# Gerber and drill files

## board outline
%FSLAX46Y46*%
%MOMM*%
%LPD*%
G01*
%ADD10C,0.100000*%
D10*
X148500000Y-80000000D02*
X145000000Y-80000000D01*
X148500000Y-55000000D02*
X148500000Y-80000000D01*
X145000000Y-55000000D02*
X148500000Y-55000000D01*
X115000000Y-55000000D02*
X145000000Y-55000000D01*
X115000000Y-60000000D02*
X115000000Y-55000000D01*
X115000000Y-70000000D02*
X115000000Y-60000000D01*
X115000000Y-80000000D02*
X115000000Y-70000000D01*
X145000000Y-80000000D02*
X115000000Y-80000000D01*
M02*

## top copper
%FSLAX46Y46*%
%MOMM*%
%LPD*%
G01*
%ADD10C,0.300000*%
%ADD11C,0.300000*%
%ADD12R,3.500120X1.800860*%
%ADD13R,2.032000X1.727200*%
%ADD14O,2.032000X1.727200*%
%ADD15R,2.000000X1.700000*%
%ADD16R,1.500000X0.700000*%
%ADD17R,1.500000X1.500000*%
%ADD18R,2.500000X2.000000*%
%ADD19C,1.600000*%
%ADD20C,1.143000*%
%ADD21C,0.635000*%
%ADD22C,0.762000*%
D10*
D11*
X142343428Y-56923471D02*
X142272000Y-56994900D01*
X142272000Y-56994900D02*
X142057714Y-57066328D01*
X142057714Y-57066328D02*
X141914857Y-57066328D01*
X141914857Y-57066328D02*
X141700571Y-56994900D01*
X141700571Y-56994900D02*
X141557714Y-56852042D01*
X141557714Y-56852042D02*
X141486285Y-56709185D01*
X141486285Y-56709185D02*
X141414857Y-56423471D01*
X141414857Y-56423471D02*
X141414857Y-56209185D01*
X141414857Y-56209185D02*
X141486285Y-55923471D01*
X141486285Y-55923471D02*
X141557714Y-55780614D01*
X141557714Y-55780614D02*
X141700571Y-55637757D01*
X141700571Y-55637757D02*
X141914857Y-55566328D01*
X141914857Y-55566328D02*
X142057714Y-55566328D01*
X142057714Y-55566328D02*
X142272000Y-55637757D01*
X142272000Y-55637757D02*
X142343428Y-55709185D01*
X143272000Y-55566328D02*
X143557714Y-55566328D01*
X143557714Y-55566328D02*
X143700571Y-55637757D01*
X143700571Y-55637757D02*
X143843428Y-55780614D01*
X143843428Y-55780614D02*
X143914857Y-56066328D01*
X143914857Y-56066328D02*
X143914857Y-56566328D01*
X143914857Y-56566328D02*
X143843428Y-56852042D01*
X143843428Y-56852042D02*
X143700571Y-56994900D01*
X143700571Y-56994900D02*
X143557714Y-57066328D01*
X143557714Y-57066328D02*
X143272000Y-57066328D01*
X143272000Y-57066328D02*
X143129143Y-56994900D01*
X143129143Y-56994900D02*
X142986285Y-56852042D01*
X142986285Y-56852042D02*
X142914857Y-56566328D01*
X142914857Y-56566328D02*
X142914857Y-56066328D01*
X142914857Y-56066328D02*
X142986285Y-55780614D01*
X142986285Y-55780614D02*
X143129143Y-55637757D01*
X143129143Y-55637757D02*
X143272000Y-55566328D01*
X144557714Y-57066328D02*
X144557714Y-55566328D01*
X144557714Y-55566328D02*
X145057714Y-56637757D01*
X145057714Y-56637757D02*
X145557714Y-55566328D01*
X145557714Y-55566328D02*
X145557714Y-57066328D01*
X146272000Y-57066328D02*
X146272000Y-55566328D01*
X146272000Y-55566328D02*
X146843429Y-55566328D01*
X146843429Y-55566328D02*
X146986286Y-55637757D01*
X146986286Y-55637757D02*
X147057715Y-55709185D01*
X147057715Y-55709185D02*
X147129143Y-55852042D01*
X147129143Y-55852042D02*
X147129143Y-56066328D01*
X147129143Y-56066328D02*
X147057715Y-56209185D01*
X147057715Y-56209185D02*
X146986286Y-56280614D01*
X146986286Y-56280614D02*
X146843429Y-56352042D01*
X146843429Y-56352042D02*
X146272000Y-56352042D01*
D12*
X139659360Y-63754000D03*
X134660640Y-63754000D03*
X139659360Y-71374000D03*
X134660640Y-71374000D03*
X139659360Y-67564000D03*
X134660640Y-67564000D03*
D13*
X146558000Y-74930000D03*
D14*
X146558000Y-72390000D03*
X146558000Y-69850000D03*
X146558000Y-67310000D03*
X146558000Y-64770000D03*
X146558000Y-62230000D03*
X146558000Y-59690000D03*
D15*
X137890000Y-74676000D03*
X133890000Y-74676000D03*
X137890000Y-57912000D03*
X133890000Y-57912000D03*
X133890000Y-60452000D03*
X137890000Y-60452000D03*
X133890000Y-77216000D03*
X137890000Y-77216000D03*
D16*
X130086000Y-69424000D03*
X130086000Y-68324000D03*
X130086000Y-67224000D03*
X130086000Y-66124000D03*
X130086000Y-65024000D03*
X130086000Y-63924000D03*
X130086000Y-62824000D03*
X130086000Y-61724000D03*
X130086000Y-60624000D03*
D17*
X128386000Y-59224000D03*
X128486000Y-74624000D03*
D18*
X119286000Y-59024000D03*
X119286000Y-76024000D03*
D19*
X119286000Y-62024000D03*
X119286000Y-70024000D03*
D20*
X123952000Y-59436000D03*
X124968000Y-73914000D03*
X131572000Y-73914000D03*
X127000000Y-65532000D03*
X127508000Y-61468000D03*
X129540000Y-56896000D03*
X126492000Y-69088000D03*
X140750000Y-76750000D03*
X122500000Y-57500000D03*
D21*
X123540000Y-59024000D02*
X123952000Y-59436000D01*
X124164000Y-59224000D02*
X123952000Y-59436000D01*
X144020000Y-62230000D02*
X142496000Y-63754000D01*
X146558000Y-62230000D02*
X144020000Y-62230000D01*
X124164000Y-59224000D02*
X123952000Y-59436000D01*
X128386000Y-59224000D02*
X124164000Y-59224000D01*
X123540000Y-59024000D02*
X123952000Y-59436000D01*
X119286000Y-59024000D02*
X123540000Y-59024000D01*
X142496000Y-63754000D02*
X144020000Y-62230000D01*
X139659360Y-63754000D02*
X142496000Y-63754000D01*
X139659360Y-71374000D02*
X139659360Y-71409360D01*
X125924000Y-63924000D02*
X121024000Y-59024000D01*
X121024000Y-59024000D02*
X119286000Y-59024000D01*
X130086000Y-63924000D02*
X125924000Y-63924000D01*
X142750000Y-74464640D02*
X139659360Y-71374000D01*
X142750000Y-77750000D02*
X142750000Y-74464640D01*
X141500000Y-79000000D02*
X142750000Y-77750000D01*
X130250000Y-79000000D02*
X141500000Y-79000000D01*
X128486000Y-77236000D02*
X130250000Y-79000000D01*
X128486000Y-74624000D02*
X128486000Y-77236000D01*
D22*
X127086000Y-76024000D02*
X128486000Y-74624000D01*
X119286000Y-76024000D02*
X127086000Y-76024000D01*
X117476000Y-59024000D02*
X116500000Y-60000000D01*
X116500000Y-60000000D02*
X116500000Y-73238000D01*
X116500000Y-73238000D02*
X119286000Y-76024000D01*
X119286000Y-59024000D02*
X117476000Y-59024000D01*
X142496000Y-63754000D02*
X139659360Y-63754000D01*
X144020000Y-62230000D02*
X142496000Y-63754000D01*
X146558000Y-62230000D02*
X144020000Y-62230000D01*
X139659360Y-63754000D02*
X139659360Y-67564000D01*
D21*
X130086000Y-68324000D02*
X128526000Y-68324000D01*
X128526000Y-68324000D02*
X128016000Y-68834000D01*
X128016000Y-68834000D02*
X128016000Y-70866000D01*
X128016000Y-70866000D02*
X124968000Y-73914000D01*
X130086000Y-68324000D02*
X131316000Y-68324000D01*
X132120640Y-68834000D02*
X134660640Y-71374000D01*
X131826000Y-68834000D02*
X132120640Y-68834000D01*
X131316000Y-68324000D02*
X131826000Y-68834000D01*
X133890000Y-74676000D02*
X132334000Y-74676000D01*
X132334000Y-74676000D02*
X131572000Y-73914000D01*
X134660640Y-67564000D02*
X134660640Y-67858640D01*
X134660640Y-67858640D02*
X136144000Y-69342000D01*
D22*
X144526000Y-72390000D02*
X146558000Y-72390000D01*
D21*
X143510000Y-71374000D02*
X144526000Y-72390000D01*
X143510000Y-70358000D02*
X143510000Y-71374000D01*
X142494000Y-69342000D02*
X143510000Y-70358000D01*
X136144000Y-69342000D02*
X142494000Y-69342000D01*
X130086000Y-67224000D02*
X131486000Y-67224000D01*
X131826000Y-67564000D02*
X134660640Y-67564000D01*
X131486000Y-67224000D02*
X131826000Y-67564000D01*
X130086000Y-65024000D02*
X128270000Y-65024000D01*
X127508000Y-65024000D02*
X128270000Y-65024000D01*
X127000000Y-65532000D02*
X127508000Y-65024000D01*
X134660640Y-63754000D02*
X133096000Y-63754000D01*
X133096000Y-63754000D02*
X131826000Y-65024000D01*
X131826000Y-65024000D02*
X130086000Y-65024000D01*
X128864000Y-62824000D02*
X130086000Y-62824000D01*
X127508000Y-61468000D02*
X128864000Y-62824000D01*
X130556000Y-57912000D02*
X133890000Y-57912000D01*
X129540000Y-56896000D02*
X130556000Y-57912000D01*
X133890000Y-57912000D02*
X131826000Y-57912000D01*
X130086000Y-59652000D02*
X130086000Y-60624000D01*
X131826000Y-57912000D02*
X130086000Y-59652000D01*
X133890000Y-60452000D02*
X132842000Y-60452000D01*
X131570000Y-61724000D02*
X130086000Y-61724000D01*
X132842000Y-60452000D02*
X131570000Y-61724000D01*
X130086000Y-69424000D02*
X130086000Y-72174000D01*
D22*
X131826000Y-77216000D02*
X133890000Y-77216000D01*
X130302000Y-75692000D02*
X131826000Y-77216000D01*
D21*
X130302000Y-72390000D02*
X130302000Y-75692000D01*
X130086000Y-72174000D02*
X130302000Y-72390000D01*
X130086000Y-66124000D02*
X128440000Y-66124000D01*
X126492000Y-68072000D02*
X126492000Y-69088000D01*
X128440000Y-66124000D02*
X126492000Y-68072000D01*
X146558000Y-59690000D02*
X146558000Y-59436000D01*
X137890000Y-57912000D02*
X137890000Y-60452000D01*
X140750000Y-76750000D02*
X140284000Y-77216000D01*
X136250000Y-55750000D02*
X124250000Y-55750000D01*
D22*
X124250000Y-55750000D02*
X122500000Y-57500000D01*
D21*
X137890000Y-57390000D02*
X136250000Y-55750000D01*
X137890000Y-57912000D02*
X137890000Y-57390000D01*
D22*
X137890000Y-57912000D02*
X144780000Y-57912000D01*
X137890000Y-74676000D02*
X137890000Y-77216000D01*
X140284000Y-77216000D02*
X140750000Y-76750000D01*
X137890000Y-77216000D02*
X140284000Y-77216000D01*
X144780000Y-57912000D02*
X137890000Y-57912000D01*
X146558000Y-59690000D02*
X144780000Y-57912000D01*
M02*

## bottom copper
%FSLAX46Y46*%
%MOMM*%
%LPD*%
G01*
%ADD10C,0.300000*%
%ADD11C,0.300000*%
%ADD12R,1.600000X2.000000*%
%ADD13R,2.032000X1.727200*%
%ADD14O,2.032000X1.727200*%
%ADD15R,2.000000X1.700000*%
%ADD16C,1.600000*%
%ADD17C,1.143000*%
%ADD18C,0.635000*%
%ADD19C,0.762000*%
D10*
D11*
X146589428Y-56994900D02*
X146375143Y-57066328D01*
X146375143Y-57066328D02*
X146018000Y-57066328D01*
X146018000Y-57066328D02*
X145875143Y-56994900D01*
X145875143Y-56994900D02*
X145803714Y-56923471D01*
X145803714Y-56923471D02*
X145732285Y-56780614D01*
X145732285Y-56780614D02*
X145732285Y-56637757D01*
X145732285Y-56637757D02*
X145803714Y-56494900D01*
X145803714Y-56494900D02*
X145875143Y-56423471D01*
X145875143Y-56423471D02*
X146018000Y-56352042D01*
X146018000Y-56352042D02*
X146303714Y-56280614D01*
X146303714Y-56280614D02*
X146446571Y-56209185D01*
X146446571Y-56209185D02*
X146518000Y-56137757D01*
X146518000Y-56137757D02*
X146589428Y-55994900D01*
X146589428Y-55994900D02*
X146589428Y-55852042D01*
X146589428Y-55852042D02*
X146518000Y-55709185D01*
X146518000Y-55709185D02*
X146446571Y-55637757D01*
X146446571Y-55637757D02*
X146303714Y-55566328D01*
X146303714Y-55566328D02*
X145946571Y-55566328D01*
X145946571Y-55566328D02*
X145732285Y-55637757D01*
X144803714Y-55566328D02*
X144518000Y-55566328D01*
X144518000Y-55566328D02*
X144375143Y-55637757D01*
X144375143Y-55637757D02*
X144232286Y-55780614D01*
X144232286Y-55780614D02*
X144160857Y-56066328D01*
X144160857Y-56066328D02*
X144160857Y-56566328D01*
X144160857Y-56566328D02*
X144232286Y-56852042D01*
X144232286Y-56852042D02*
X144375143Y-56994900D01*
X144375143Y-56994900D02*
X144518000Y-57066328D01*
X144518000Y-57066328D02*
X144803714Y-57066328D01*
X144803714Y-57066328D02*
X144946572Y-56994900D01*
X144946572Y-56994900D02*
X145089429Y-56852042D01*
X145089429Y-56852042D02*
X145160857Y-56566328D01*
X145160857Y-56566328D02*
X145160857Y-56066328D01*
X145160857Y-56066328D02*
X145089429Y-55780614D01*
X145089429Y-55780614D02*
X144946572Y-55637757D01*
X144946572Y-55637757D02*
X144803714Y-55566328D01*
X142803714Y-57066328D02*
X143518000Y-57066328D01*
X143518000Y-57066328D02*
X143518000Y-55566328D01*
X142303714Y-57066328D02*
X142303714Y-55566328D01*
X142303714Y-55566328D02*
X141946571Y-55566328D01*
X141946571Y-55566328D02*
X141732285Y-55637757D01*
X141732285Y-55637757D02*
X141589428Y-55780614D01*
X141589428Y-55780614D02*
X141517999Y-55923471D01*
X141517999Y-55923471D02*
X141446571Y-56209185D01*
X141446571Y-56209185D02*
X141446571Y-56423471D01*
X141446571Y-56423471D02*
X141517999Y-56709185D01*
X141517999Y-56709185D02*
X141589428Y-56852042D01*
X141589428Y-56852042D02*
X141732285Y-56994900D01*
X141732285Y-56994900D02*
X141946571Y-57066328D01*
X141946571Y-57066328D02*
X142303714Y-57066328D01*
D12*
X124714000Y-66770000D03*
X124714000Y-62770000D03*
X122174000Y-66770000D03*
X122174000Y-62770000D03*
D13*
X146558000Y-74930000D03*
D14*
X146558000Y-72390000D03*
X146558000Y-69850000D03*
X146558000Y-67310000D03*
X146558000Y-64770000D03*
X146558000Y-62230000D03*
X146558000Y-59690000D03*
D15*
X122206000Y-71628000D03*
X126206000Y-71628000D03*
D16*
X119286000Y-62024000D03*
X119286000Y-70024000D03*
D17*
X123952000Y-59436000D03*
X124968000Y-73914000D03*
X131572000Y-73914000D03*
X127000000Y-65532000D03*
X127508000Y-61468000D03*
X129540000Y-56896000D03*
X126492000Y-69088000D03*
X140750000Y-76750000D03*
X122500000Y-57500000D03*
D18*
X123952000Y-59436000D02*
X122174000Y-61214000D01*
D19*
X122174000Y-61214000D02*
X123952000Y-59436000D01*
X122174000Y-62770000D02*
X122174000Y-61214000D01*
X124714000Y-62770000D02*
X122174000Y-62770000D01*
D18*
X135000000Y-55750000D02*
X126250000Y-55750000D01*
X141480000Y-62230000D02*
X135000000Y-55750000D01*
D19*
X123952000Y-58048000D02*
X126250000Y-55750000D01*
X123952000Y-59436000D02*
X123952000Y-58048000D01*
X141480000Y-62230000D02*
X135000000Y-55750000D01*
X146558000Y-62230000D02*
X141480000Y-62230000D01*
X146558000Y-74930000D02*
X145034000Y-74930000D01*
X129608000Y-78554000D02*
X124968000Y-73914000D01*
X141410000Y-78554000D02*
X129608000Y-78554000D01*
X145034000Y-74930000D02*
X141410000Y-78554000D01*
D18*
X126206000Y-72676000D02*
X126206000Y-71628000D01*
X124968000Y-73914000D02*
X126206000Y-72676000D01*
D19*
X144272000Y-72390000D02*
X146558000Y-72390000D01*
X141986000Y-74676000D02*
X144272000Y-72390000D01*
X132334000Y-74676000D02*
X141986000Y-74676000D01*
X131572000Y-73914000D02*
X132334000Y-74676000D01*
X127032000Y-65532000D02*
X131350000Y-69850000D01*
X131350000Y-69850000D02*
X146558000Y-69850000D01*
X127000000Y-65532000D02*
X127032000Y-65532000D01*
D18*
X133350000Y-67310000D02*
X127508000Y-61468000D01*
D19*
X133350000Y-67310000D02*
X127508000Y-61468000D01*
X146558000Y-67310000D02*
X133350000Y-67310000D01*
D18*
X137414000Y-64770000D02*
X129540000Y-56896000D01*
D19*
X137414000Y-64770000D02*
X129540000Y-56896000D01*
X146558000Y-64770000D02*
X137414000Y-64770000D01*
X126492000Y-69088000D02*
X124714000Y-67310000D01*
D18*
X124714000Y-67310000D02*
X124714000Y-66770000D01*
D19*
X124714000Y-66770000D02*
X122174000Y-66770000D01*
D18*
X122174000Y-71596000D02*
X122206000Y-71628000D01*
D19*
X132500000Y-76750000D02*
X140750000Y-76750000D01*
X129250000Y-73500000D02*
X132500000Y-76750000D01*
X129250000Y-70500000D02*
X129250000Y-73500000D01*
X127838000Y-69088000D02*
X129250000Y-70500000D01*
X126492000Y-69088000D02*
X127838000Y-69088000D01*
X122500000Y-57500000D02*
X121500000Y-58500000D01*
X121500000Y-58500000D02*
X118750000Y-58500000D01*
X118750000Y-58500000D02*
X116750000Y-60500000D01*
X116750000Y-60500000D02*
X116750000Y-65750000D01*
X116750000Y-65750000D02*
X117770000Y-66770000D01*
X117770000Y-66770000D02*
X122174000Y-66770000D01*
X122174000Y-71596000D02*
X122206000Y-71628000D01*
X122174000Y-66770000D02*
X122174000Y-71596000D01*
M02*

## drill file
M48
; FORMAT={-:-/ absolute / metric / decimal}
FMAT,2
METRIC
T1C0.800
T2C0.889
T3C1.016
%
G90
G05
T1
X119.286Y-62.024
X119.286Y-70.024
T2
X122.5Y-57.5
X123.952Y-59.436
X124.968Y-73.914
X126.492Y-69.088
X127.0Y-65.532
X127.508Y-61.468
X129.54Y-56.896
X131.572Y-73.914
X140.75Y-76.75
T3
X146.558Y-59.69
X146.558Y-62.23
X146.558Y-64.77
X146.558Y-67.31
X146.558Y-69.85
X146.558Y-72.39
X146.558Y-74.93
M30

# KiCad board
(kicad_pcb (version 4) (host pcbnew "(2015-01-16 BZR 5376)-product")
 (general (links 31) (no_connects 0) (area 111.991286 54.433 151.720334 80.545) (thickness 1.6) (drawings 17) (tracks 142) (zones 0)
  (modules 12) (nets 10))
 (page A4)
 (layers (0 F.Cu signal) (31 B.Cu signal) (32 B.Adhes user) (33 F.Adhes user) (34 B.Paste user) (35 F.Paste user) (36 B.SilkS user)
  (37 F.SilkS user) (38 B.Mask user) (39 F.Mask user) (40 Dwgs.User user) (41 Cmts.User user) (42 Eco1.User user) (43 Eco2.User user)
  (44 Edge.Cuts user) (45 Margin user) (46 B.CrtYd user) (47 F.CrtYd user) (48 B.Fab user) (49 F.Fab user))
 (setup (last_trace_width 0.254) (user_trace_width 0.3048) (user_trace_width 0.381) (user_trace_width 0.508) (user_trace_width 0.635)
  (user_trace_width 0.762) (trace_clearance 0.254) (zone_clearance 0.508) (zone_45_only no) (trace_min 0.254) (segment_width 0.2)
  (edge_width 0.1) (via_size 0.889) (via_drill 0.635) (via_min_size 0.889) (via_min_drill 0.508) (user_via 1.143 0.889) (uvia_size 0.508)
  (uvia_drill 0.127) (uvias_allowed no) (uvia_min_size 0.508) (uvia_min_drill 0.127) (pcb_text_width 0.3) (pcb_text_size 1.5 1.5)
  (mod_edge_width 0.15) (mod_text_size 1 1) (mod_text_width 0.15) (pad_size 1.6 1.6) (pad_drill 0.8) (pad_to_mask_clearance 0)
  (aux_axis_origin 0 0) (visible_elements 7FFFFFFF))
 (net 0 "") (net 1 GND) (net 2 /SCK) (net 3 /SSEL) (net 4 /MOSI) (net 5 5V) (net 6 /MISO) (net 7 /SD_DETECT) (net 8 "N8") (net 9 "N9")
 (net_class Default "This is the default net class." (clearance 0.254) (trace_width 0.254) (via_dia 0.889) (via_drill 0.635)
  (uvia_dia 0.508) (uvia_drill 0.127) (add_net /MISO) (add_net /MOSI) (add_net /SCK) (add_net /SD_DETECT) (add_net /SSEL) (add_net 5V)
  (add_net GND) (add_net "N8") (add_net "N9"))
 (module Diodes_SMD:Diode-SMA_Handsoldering (layer F.Cu) (at 137.16 63.754 180)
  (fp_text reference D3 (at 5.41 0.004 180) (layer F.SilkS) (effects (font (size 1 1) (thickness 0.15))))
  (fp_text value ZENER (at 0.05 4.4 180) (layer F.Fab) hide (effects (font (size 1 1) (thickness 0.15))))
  (pad 1 smd rect (at -2.49936 0 180) (size 3.50012 1.80086) (layers F.Cu F.Paste F.Mask) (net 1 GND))
  (pad 2 smd rect (at 2.49936 0 180) (size 3.50012 1.80086) (layers F.Cu F.Paste F.Mask) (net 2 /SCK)))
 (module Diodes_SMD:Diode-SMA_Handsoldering (layer F.Cu) (at 137.16 71.374 180)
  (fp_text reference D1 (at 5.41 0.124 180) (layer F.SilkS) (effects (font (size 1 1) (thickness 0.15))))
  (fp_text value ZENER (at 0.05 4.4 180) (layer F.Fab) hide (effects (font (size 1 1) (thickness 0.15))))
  (pad 1 smd rect (at -2.49936 0 180) (size 3.50012 1.80086) (layers F.Cu F.Paste F.Mask) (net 1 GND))
  (pad 2 smd rect (at 2.49936 0 180) (size 3.50012 1.80086) (layers F.Cu F.Paste F.Mask) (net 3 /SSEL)))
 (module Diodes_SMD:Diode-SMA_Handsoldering (layer F.Cu) (at 137.16 67.564 180)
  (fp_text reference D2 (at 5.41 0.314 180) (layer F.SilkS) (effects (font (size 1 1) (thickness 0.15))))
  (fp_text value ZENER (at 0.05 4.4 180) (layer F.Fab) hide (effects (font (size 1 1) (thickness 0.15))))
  (pad 1 smd rect (at -2.49936 0 180) (size 3.50012 1.80086) (layers F.Cu F.Paste F.Mask) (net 1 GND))
  (pad 2 smd rect (at 2.49936 0 180) (size 3.50012 1.80086) (layers F.Cu F.Paste F.Mask) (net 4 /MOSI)))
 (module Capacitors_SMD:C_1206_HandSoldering (layer B.Cu) (at 124.714 64.77 90)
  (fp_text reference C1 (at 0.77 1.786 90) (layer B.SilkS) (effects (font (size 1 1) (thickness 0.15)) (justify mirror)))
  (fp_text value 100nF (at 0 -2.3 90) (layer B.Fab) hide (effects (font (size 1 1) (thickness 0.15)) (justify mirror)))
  (pad 1 smd rect (at -2 0 90) (size 2 1.6) (layers B.Cu B.Paste B.Mask) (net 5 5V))
  (pad 2 smd rect (at 2 0 90) (size 2 1.6) (layers B.Cu B.Paste B.Mask) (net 1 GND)))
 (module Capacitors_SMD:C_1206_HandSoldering (layer B.Cu) (at 122.174 64.77 90)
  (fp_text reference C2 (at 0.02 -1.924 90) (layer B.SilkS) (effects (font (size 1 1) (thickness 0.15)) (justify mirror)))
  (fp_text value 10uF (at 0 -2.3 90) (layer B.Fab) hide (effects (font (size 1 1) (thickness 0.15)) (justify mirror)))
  (pad 1 smd rect (at -2 0 90) (size 2 1.6) (layers B.Cu B.Paste B.Mask) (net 5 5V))
  (pad 2 smd rect (at 2 0 90) (size 2 1.6) (layers B.Cu B.Paste B.Mask) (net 1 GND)))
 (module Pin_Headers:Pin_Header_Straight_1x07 (layer F.Cu) (at 146.558 74.93 180)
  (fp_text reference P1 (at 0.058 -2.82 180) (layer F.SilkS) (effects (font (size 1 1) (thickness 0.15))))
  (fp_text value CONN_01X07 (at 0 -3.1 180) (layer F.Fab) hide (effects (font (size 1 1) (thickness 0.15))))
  (pad 1 thru_hole rect (at 0 0 180) (size 2.032 1.7272) (drill 1.016) (layers *.Cu *.Mask F.SilkS) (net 3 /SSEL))
  (pad 2 thru_hole oval (at 0 2.54 180) (size 2.032 1.7272) (drill 1.016) (layers *.Cu *.Mask F.SilkS) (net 4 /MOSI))
  (pad 3 thru_hole oval (at 0 5.08 180) (size 2.032 1.7272) (drill 1.016) (layers *.Cu *.Mask F.SilkS) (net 2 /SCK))
  (pad 4 thru_hole oval (at 0 7.62 180) (size 2.032 1.7272) (drill 1.016) (layers *.Cu *.Mask F.SilkS) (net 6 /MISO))
  (pad 5 thru_hole oval (at 0 10.16 180) (size 2.032 1.7272) (drill 1.016) (layers *.Cu *.Mask F.SilkS) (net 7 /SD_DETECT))
  (pad 6 thru_hole oval (at 0 12.7 180) (size 2.032 1.7272) (drill 1.016) (layers *.Cu *.Mask F.SilkS) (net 1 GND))
  (pad 7 thru_hole oval (at 0 15.24 180) (size 2.032 1.7272) (drill 1.016) (layers *.Cu *.Mask F.SilkS) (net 5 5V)))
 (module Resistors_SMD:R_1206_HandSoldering (layer B.Cu) (at 124.206 71.628)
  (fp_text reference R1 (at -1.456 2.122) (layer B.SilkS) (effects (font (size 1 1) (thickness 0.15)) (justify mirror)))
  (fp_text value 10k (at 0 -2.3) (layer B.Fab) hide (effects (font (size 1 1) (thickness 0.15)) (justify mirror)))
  (pad 1 smd rect (at -2 0) (size 2 1.7) (layers B.Cu B.Paste B.Mask) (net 5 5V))
  (pad 2 smd rect (at 2 0) (size 2 1.7) (layers B.Cu B.Paste B.Mask) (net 3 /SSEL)))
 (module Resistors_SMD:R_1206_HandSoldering (layer F.Cu) (at 135.89 74.676 180)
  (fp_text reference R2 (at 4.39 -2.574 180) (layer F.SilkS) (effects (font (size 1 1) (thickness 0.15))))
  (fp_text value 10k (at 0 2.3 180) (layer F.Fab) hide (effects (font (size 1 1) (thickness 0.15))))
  (pad 1 smd rect (at -2 0 180) (size 2 1.7) (layers F.Cu F.Paste F.Mask) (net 5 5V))
  (pad 2 smd rect (at 2 0 180) (size 2 1.7) (layers F.Cu F.Paste F.Mask) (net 4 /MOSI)))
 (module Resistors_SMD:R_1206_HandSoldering (layer F.Cu) (at 135.89 57.912 180)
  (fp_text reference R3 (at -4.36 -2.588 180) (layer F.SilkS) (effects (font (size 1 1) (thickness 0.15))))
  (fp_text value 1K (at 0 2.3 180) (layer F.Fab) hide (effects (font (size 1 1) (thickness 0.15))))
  (pad 1 smd rect (at -2 0 180) (size 2 1.7) (layers F.Cu F.Paste F.Mask) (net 5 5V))
  (pad 2 smd rect (at 2 0 180) (size 2 1.7) (layers F.Cu F.Paste F.Mask) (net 7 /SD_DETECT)))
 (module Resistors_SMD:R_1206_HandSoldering (layer F.Cu) (at 135.89 60.452)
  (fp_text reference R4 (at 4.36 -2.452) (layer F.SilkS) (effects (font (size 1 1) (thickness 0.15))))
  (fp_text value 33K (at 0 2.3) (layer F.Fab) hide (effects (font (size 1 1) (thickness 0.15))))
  (pad 1 smd rect (at -2 0) (size 2 1.7) (layers F.Cu F.Paste F.Mask) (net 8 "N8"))
  (pad 2 smd rect (at 2 0) (size 2 1.7) (layers F.Cu F.Paste F.Mask) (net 5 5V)))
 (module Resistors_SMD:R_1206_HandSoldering (layer F.Cu) (at 135.89 77.216)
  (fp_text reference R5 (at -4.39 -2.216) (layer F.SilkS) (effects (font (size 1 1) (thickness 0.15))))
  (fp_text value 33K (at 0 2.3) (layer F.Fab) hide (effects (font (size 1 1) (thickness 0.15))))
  (pad 1 smd rect (at -2 0) (size 2 1.7) (layers F.Cu F.Paste F.Mask) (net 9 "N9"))
  (pad 2 smd rect (at 2 0) (size 2 1.7) (layers F.Cu F.Paste F.Mask) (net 5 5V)))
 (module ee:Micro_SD (layer F.Cu) (at 129.286 65.024 270)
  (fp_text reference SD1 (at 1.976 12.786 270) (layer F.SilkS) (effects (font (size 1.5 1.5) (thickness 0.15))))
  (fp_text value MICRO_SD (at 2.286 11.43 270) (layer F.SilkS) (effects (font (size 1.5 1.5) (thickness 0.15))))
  (pad 1 smd rect (at 4.4 -0.8 270) (size 0.7 1.5) (layers F.Cu F.Paste F.Mask) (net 9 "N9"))
  (pad 2 smd rect (at 3.3 -0.8 270) (size 0.7 1.5) (layers F.Cu F.Paste F.Mask) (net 3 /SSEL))
  (pad 3 smd rect (at 2.2 -0.8 270) (size 0.7 1.5) (layers F.Cu F.Paste F.Mask) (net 4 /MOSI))
  (pad 4 smd rect (at 1.1 -0.8 270) (size 0.7 1.5) (layers F.Cu F.Paste F.Mask) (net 5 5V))
  (pad 5 smd rect (at 0 -0.8 270) (size 0.7 1.5) (layers F.Cu F.Paste F.Mask) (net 2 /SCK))
  (pad 6 smd rect (at -1.1 -0.8 270) (size 0.7 1.5) (layers F.Cu F.Paste F.Mask) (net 1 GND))
  (pad 7 smd rect (at -2.2 -0.8 270) (size 0.7 1.5) (layers F.Cu F.Paste F.Mask) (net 6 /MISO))
  (pad 8 smd rect (at -3.3 -0.8 270) (size 0.7 1.5) (layers F.Cu F.Paste F.Mask) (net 8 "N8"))
  (pad 9 smd rect (at -4.4 -0.8 270) (size 0.7 1.5) (layers F.Cu F.Paste F.Mask) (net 7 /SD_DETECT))
  (pad 10 smd rect (at -5.8 0.9 270) (size 1.5 1.5) (layers F.Cu F.Paste F.Mask) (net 1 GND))
  (pad 11 smd rect (at 9.6 0.8 270) (size 1.5 1.5) (layers F.Cu F.Paste F.Mask) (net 1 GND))
  (pad 12 smd rect (at -6 10 270) (size 2 2.5) (layers F.Cu F.Paste F.Mask) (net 1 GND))
  (pad 13 smd rect (at 11 10 270) (size 2 2.5) (layers F.Cu F.Paste F.Mask) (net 1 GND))
  (pad "" thru_hole circle (at -3 10 270) (size 1.6 1.6) (drill 0.8) (layers *.Cu *.Mask F.SilkS))
  (pad "" thru_hole circle (at 5 10 270) (size 1.6 1.6) (drill 0.8) (layers *.Cu *.Mask F.SilkS)))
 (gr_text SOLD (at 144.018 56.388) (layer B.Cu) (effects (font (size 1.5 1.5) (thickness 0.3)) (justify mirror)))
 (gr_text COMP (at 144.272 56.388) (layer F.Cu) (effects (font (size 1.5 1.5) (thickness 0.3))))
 (gr_line (start 148.5 80) (end 145 80) (angle 90) (layer Edge.Cuts) (width 0.1))
 (gr_line (start 148.5 55) (end 148.5 80) (angle 90) (layer Edge.Cuts) (width 0.1))
 (gr_line (start 145 55) (end 148.5 55) (angle 90) (layer Edge.Cuts) (width 0.1))
 (gr_line (start 115 55) (end 145 55) (angle 90) (layer Edge.Cuts) (width 0.1))
 (gr_line (start 115 60) (end 115 55) (angle 90) (layer Edge.Cuts) (width 0.1))
 (gr_line (start 115 70) (end 115 60) (angle 90) (layer Edge.Cuts) (width 0.1))
 (gr_line (start 115 80) (end 115 70) (angle 90) (layer Edge.Cuts) (width 0.1))
 (gr_line (start 145 80) (end 115 80) (angle 90) (layer Edge.Cuts) (width 0.1))
 (segment (start 123.54 59.024) (end 123.952 59.436) (width 0.635) (layer F.Cu) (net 1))
 (segment (start 124.164 59.224) (end 123.952 59.436) (width 0.635) (layer F.Cu) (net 1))
 (via (at 123.952 59.436) (size 1.143) (drill 0.889) (layers F.Cu B.Cu) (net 1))
 (segment (start 123.952 59.436) (end 122.174 61.214) (width 0.635) (layer B.Cu) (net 1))
 (segment (start 144.02 62.23) (end 142.496 63.754) (width 0.635) (layer F.Cu) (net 1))
 (segment (start 146.558 62.23) (end 144.02 62.23) (width 0.635) (layer F.Cu) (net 1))
 (segment (start 124.164 59.224) (end 123.952 59.436) (width 0.635) (layer F.Cu) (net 1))
 (segment (start 128.386 59.224) (end 124.164 59.224) (width 0.635) (layer F.Cu) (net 1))
 (segment (start 123.54 59.024) (end 123.952 59.436) (width 0.635) (layer F.Cu) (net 1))
 (segment (start 119.286 59.024) (end 123.54 59.024) (width 0.635) (layer F.Cu) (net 1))
 (segment (start 122.174 61.214) (end 123.952 59.436) (width 0.762) (layer B.Cu) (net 1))
 (segment (start 122.174 62.77) (end 122.174 61.214) (width 0.762) (layer B.Cu) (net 1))
 (segment (start 124.714 62.77) (end 122.174 62.77) (width 0.762) (layer B.Cu) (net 1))
 (segment (start 142.496 63.754) (end 144.02 62.23) (width 0.635) (layer F.Cu) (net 1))
 (segment (start 139.65936 63.754) (end 142.496 63.754) (width 0.635) (layer F.Cu) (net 1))
 (segment (start 139.65936 71.374) (end 139.65936 71.40936) (width 0.635) (layer F.Cu) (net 1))
 (segment (start 125.924 63.924) (end 121.024 59.024) (width 0.635) (layer F.Cu) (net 1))
 (segment (start 121.024 59.024) (end 119.286 59.024) (width 0.635) (layer F.Cu) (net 1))
 (segment (start 130.086 63.924) (end 125.924 63.924) (width 0.635) (layer F.Cu) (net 1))
 (segment (start 142.75 74.46464) (end 139.65936 71.374) (width 0.635) (layer F.Cu) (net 1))
 (segment (start 142.75 77.75) (end 142.75 74.46464) (width 0.635) (layer F.Cu) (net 1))
 (segment (start 141.5 79) (end 142.75 77.75) (width 0.635) (layer F.Cu) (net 1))
 (segment (start 130.25 79) (end 141.5 79) (width 0.635) (layer F.Cu) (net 1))
 (segment (start 128.486 77.236) (end 130.25 79) (width 0.635) (layer F.Cu) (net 1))
 (segment (start 128.486 74.624) (end 128.486 77.236) (width 0.635) (layer F.Cu) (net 1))
 (segment (start 127.086 76.024) (end 128.486 74.624) (width 0.762) (layer F.Cu) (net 1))
 (segment (start 119.286 76.024) (end 127.086 76.024) (width 0.762) (layer F.Cu) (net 1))
 (segment (start 117.476 59.024) (end 116.5 60) (width 0.762) (layer F.Cu) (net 1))
 (segment (start 116.5 60) (end 116.5 73.238) (width 0.762) (layer F.Cu) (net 1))
 (segment (start 116.5 73.238) (end 119.286 76.024) (width 0.762) (layer F.Cu) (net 1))
 (segment (start 119.286 59.024) (end 117.476 59.024) (width 0.762) (layer F.Cu) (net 1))
 (segment (start 142.496 63.754) (end 139.65936 63.754) (width 0.762) (layer F.Cu) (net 1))
 (segment (start 144.02 62.23) (end 142.496 63.754) (width 0.762) (layer F.Cu) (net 1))
 (segment (start 146.558 62.23) (end 144.02 62.23) (width 0.762) (layer F.Cu) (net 1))
 (segment (start 139.65936 63.754) (end 139.65936 67.564) (width 0.762) (layer F.Cu) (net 1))
 (segment (start 135 55.75) (end 126.25 55.75) (width 0.635) (layer B.Cu) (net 1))
 (segment (start 141.48 62.23) (end 135 55.75) (width 0.635) (layer B.Cu) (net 1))
 (segment (start 123.952 58.048) (end 126.25 55.75) (width 0.762) (layer B.Cu) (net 1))
 (segment (start 123.952 59.436) (end 123.952 58.048) (width 0.762) (layer B.Cu) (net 1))
 (segment (start 141.48 62.23) (end 135 55.75) (width 0.762) (layer B.Cu) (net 1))
 (segment (start 146.558 62.23) (end 141.48 62.23) (width 0.762) (layer B.Cu) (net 1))
 (segment (start 146.558 74.93) (end 145.034 74.93) (width 0.762) (layer B.Cu) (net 3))
 (segment (start 129.608 78.554) (end 124.968 73.914) (width 0.762) (layer B.Cu) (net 3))
 (segment (start 141.41 78.554) (end 129.608 78.554) (width 0.762) (layer B.Cu) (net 3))
 (segment (start 145.034 74.93) (end 141.41 78.554) (width 0.762) (layer B.Cu) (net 3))
 (segment (start 130.086 68.324) (end 128.526 68.324) (width 0.635) (layer F.Cu) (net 3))
 (segment (start 128.526 68.324) (end 128.016 68.834) (width 0.635) (layer F.Cu) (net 3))
 (segment (start 128.016 68.834) (end 128.016 70.866) (width 0.635) (layer F.Cu) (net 3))
 (segment (start 128.016 70.866) (end 124.968 73.914) (width 0.635) (layer F.Cu) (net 3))
 (via (at 124.968 73.914) (size 1.143) (drill 0.889) (layers F.Cu B.Cu) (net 3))
 (segment (start 126.206 72.676) (end 126.206 71.628) (width 0.635) (layer B.Cu) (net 3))
 (segment (start 124.968 73.914) (end 126.206 72.676) (width 0.635) (layer B.Cu) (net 3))
 (segment (start 130.086 68.324) (end 131.316 68.324) (width 0.635) (layer F.Cu) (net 3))
 (segment (start 132.12064 68.834) (end 134.66064 71.374) (width 0.635) (layer F.Cu) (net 3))
 (segment (start 131.826 68.834) (end 132.12064 68.834) (width 0.635) (layer F.Cu) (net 3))
 (segment (start 131.316 68.324) (end 131.826 68.834) (width 0.635) (layer F.Cu) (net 3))
 (segment (start 133.89 74.676) (end 132.334 74.676) (width 0.635) (layer F.Cu) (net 4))
 (segment (start 144.272 72.39) (end 146.558 72.39) (width 0.762) (layer B.Cu) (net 4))
 (segment (start 141.986 74.676) (end 144.272 72.39) (width 0.762) (layer B.Cu) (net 4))
 (segment (start 132.334 74.676) (end 141.986 74.676) (width 0.762) (layer B.Cu) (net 4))
 (segment (start 131.572 73.914) (end 132.334 74.676) (width 0.762) (layer B.Cu) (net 4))
 (via (at 131.572 73.914) (size 1.143) (drill 0.889) (layers F.Cu B.Cu) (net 4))
 (segment (start 132.334 74.676) (end 131.572 73.914) (width 0.635) (layer F.Cu) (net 4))
 (segment (start 134.66064 67.564) (end 134.66064 67.85864) (width 0.635) (layer F.Cu) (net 4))
 (segment (start 134.66064 67.85864) (end 136.144 69.342) (width 0.635) (layer F.Cu) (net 4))
 (segment (start 144.526 72.39) (end 146.558 72.39) (width 0.762) (layer F.Cu) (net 4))
 (segment (start 143.51 71.374) (end 144.526 72.39) (width 0.635) (layer F.Cu) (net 4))
 (segment (start 143.51 70.358) (end 143.51 71.374) (width 0.635) (layer F.Cu) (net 4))
 (segment (start 142.494 69.342) (end 143.51 70.358) (width 0.635) (layer F.Cu) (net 4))
 (segment (start 136.144 69.342) (end 142.494 69.342) (width 0.635) (layer F.Cu) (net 4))
 (segment (start 130.086 67.224) (end 131.486 67.224) (width 0.635) (layer F.Cu) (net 4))
 (segment (start 131.826 67.564) (end 134.66064 67.564) (width 0.635) (layer F.Cu) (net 4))
 (segment (start 131.486 67.224) (end 131.826 67.564) (width 0.635) (layer F.Cu) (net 4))
 (segment (start 130.086 65.024) (end 128.27 65.024) (width 0.635) (layer F.Cu) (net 2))
 (segment (start 127.508 65.024) (end 128.27 65.024) (width 0.635) (layer F.Cu) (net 2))
 (segment (start 127 65.532) (end 127.508 65.024) (width 0.635) (layer F.Cu) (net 2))
 (via (at 127 65.532) (size 1.143) (drill 0.889) (layers F.Cu B.Cu) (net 2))
 (segment (start 134.66064 63.754) (end 133.096 63.754) (width 0.635) (layer F.Cu) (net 2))
 (segment (start 133.096 63.754) (end 131.826 65.024) (width 0.635) (layer F.Cu) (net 2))
 (segment (start 131.826 65.024) (end 130.086 65.024) (width 0.635) (layer F.Cu) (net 2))
 (segment (start 127.032 65.532) (end 131.35 69.85) (width 0.762) (layer B.Cu) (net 2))
 (segment (start 131.35 69.85) (end 146.558 69.85) (width 0.762) (layer B.Cu) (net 2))
 (segment (start 127 65.532) (end 127.032 65.532) (width 0.762) (layer B.Cu) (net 2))
 (segment (start 128.864 62.824) (end 130.086 62.824) (width 0.635) (layer F.Cu) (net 6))
 (segment (start 127.508 61.468) (end 128.864 62.824) (width 0.635) (layer F.Cu) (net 6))
 (via (at 127.508 61.468) (size 1.143) (drill 0.889) (layers F.Cu B.Cu) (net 6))
 (segment (start 133.35 67.31) (end 127.508 61.468) (width 0.635) (layer B.Cu) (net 6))
 (segment (start 133.35 67.31) (end 127.508 61.468) (width 0.762) (layer B.Cu) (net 6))
 (segment (start 146.558 67.31) (end 133.35 67.31) (width 0.762) (layer B.Cu) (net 6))
 (segment (start 130.556 57.912) (end 133.89 57.912) (width 0.635) (layer F.Cu) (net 7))
 (segment (start 129.54 56.896) (end 130.556 57.912) (width 0.635) (layer F.Cu) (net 7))
 (via (at 129.54 56.896) (size 1.143) (drill 0.889) (layers F.Cu B.Cu) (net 7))
 (segment (start 137.414 64.77) (end 129.54 56.896) (width 0.635) (layer B.Cu) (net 7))
 (segment (start 133.89 57.912) (end 131.826 57.912) (width 0.635) (layer F.Cu) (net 7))
 (segment (start 130.086 59.652) (end 130.086 60.624) (width 0.635) (layer F.Cu) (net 7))
 (segment (start 131.826 57.912) (end 130.086 59.652) (width 0.635) (layer F.Cu) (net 7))
 (segment (start 137.414 64.77) (end 129.54 56.896) (width 0.762) (layer B.Cu) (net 7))
 (segment (start 146.558 64.77) (end 137.414 64.77) (width 0.762) (layer B.Cu) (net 7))
 (segment (start 133.89 60.452) (end 132.842 60.452) (width 0.635) (layer F.Cu) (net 8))
 (segment (start 131.57 61.724) (end 130.086 61.724) (width 0.635) (layer F.Cu) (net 8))
 (segment (start 132.842 60.452) (end 131.57 61.724) (width 0.635) (layer F.Cu) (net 8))
 (segment (start 130.086 69.424) (end 130.086 72.174) (width 0.635) (layer F.Cu) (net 9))
 (segment (start 131.826 77.216) (end 133.89 77.216) (width 0.762) (layer F.Cu) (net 9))
 (segment (start 130.302 75.692) (end 131.826 77.216) (width 0.762) (layer F.Cu) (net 9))
 (segment (start 130.302 72.39) (end 130.302 75.692) (width 0.635) (layer F.Cu) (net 9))
 (segment (start 130.086 72.174) (end 130.302 72.39) (width 0.635) (layer F.Cu) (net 9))
 (segment (start 130.086 66.124) (end 128.44 66.124) (width 0.635) (layer F.Cu) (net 5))
 (segment (start 126.492 69.088) (end 124.714 67.31) (width 0.762) (layer B.Cu) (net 5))
 (via (at 126.492 69.088) (size 1.143) (drill 0.889) (layers F.Cu B.Cu) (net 5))
 (segment (start 126.492 68.072) (end 126.492 69.088) (width 0.635) (layer F.Cu) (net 5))
 (segment (start 128.44 66.124) (end 126.492 68.072) (width 0.635) (layer F.Cu) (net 5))
 (segment (start 124.714 67.31) (end 124.714 66.77) (width 0.635) (layer B.Cu) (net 5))
 (segment (start 146.558 59.69) (end 146.558 59.436) (width 0.635) (layer F.Cu) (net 5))
 (segment (start 124.714 66.77) (end 122.174 66.77) (width 0.762) (layer B.Cu) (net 5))
 (segment (start 137.89 57.912) (end 137.89 60.452) (width 0.635) (layer F.Cu) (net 5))
 (segment (start 122.174 71.596) (end 122.206 71.628) (width 0.635) (layer B.Cu) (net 5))
 (segment (start 140.75 76.75) (end 140.284 77.216) (width 0.635) (layer F.Cu) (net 5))
 (via (at 140.75 76.75) (size 1.143) (drill 0.889) (layers F.Cu B.Cu) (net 5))
 (segment (start 132.5 76.75) (end 140.75 76.75) (width 0.762) (layer B.Cu) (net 5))
 (segment (start 129.25 73.5) (end 132.5 76.75) (width 0.762) (layer B.Cu) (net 5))
 (segment (start 129.25 70.5) (end 129.25 73.5) (width 0.762) (layer B.Cu) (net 5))
 (segment (start 127.838 69.088) (end 129.25 70.5) (width 0.762) (layer B.Cu) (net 5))
 (segment (start 126.492 69.088) (end 127.838 69.088) (width 0.762) (layer B.Cu) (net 5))
 (segment (start 136.25 55.75) (end 124.25 55.75) (width 0.635) (layer F.Cu) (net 5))
 (segment (start 124.25 55.75) (end 122.5 57.5) (width 0.762) (layer F.Cu) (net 5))
 (via (at 122.5 57.5) (size 1.143) (drill 0.889) (layers F.Cu B.Cu) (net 5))
 (segment (start 122.5 57.5) (end 121.5 58.5) (width 0.762) (layer B.Cu) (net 5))
 (segment (start 121.5 58.5) (end 118.75 58.5) (width 0.762) (layer B.Cu) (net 5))
 (segment (start 118.75 58.5) (end 116.75 60.5) (width 0.762) (layer B.Cu) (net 5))
 (segment (start 116.75 60.5) (end 116.75 65.75) (width 0.762) (layer B.Cu) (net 5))
 (segment (start 116.75 65.75) (end 117.77 66.77) (width 0.762) (layer B.Cu) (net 5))
 (segment (start 117.77 66.77) (end 122.174 66.77) (width 0.762) (layer B.Cu) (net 5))
 (segment (start 137.89 57.39) (end 136.25 55.75) (width 0.635) (layer F.Cu) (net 5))
 (segment (start 137.89 57.912) (end 137.89 57.39) (width 0.635) (layer F.Cu) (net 5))
 (segment (start 137.89 57.912) (end 144.78 57.912) (width 0.762) (layer F.Cu) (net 5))
 (segment (start 137.89 74.676) (end 137.89 77.216) (width 0.762) (layer F.Cu) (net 5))
 (segment (start 140.284 77.216) (end 140.75 76.75) (width 0.762) (layer F.Cu) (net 5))
 (segment (start 137.89 77.216) (end 140.284 77.216) (width 0.762) (layer F.Cu) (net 5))
 (segment (start 144.78 57.912) (end 137.89 57.912) (width 0.762) (layer F.Cu) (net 5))
 (segment (start 146.558 59.69) (end 144.78 57.912) (width 0.762) (layer F.Cu) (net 5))
 (segment (start 122.174 71.596) (end 122.206 71.628) (width 0.762) (layer B.Cu) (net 5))
 (segment (start 122.174 66.77) (end 122.174 71.596) (width 0.762) (layer B.Cu) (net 5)))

